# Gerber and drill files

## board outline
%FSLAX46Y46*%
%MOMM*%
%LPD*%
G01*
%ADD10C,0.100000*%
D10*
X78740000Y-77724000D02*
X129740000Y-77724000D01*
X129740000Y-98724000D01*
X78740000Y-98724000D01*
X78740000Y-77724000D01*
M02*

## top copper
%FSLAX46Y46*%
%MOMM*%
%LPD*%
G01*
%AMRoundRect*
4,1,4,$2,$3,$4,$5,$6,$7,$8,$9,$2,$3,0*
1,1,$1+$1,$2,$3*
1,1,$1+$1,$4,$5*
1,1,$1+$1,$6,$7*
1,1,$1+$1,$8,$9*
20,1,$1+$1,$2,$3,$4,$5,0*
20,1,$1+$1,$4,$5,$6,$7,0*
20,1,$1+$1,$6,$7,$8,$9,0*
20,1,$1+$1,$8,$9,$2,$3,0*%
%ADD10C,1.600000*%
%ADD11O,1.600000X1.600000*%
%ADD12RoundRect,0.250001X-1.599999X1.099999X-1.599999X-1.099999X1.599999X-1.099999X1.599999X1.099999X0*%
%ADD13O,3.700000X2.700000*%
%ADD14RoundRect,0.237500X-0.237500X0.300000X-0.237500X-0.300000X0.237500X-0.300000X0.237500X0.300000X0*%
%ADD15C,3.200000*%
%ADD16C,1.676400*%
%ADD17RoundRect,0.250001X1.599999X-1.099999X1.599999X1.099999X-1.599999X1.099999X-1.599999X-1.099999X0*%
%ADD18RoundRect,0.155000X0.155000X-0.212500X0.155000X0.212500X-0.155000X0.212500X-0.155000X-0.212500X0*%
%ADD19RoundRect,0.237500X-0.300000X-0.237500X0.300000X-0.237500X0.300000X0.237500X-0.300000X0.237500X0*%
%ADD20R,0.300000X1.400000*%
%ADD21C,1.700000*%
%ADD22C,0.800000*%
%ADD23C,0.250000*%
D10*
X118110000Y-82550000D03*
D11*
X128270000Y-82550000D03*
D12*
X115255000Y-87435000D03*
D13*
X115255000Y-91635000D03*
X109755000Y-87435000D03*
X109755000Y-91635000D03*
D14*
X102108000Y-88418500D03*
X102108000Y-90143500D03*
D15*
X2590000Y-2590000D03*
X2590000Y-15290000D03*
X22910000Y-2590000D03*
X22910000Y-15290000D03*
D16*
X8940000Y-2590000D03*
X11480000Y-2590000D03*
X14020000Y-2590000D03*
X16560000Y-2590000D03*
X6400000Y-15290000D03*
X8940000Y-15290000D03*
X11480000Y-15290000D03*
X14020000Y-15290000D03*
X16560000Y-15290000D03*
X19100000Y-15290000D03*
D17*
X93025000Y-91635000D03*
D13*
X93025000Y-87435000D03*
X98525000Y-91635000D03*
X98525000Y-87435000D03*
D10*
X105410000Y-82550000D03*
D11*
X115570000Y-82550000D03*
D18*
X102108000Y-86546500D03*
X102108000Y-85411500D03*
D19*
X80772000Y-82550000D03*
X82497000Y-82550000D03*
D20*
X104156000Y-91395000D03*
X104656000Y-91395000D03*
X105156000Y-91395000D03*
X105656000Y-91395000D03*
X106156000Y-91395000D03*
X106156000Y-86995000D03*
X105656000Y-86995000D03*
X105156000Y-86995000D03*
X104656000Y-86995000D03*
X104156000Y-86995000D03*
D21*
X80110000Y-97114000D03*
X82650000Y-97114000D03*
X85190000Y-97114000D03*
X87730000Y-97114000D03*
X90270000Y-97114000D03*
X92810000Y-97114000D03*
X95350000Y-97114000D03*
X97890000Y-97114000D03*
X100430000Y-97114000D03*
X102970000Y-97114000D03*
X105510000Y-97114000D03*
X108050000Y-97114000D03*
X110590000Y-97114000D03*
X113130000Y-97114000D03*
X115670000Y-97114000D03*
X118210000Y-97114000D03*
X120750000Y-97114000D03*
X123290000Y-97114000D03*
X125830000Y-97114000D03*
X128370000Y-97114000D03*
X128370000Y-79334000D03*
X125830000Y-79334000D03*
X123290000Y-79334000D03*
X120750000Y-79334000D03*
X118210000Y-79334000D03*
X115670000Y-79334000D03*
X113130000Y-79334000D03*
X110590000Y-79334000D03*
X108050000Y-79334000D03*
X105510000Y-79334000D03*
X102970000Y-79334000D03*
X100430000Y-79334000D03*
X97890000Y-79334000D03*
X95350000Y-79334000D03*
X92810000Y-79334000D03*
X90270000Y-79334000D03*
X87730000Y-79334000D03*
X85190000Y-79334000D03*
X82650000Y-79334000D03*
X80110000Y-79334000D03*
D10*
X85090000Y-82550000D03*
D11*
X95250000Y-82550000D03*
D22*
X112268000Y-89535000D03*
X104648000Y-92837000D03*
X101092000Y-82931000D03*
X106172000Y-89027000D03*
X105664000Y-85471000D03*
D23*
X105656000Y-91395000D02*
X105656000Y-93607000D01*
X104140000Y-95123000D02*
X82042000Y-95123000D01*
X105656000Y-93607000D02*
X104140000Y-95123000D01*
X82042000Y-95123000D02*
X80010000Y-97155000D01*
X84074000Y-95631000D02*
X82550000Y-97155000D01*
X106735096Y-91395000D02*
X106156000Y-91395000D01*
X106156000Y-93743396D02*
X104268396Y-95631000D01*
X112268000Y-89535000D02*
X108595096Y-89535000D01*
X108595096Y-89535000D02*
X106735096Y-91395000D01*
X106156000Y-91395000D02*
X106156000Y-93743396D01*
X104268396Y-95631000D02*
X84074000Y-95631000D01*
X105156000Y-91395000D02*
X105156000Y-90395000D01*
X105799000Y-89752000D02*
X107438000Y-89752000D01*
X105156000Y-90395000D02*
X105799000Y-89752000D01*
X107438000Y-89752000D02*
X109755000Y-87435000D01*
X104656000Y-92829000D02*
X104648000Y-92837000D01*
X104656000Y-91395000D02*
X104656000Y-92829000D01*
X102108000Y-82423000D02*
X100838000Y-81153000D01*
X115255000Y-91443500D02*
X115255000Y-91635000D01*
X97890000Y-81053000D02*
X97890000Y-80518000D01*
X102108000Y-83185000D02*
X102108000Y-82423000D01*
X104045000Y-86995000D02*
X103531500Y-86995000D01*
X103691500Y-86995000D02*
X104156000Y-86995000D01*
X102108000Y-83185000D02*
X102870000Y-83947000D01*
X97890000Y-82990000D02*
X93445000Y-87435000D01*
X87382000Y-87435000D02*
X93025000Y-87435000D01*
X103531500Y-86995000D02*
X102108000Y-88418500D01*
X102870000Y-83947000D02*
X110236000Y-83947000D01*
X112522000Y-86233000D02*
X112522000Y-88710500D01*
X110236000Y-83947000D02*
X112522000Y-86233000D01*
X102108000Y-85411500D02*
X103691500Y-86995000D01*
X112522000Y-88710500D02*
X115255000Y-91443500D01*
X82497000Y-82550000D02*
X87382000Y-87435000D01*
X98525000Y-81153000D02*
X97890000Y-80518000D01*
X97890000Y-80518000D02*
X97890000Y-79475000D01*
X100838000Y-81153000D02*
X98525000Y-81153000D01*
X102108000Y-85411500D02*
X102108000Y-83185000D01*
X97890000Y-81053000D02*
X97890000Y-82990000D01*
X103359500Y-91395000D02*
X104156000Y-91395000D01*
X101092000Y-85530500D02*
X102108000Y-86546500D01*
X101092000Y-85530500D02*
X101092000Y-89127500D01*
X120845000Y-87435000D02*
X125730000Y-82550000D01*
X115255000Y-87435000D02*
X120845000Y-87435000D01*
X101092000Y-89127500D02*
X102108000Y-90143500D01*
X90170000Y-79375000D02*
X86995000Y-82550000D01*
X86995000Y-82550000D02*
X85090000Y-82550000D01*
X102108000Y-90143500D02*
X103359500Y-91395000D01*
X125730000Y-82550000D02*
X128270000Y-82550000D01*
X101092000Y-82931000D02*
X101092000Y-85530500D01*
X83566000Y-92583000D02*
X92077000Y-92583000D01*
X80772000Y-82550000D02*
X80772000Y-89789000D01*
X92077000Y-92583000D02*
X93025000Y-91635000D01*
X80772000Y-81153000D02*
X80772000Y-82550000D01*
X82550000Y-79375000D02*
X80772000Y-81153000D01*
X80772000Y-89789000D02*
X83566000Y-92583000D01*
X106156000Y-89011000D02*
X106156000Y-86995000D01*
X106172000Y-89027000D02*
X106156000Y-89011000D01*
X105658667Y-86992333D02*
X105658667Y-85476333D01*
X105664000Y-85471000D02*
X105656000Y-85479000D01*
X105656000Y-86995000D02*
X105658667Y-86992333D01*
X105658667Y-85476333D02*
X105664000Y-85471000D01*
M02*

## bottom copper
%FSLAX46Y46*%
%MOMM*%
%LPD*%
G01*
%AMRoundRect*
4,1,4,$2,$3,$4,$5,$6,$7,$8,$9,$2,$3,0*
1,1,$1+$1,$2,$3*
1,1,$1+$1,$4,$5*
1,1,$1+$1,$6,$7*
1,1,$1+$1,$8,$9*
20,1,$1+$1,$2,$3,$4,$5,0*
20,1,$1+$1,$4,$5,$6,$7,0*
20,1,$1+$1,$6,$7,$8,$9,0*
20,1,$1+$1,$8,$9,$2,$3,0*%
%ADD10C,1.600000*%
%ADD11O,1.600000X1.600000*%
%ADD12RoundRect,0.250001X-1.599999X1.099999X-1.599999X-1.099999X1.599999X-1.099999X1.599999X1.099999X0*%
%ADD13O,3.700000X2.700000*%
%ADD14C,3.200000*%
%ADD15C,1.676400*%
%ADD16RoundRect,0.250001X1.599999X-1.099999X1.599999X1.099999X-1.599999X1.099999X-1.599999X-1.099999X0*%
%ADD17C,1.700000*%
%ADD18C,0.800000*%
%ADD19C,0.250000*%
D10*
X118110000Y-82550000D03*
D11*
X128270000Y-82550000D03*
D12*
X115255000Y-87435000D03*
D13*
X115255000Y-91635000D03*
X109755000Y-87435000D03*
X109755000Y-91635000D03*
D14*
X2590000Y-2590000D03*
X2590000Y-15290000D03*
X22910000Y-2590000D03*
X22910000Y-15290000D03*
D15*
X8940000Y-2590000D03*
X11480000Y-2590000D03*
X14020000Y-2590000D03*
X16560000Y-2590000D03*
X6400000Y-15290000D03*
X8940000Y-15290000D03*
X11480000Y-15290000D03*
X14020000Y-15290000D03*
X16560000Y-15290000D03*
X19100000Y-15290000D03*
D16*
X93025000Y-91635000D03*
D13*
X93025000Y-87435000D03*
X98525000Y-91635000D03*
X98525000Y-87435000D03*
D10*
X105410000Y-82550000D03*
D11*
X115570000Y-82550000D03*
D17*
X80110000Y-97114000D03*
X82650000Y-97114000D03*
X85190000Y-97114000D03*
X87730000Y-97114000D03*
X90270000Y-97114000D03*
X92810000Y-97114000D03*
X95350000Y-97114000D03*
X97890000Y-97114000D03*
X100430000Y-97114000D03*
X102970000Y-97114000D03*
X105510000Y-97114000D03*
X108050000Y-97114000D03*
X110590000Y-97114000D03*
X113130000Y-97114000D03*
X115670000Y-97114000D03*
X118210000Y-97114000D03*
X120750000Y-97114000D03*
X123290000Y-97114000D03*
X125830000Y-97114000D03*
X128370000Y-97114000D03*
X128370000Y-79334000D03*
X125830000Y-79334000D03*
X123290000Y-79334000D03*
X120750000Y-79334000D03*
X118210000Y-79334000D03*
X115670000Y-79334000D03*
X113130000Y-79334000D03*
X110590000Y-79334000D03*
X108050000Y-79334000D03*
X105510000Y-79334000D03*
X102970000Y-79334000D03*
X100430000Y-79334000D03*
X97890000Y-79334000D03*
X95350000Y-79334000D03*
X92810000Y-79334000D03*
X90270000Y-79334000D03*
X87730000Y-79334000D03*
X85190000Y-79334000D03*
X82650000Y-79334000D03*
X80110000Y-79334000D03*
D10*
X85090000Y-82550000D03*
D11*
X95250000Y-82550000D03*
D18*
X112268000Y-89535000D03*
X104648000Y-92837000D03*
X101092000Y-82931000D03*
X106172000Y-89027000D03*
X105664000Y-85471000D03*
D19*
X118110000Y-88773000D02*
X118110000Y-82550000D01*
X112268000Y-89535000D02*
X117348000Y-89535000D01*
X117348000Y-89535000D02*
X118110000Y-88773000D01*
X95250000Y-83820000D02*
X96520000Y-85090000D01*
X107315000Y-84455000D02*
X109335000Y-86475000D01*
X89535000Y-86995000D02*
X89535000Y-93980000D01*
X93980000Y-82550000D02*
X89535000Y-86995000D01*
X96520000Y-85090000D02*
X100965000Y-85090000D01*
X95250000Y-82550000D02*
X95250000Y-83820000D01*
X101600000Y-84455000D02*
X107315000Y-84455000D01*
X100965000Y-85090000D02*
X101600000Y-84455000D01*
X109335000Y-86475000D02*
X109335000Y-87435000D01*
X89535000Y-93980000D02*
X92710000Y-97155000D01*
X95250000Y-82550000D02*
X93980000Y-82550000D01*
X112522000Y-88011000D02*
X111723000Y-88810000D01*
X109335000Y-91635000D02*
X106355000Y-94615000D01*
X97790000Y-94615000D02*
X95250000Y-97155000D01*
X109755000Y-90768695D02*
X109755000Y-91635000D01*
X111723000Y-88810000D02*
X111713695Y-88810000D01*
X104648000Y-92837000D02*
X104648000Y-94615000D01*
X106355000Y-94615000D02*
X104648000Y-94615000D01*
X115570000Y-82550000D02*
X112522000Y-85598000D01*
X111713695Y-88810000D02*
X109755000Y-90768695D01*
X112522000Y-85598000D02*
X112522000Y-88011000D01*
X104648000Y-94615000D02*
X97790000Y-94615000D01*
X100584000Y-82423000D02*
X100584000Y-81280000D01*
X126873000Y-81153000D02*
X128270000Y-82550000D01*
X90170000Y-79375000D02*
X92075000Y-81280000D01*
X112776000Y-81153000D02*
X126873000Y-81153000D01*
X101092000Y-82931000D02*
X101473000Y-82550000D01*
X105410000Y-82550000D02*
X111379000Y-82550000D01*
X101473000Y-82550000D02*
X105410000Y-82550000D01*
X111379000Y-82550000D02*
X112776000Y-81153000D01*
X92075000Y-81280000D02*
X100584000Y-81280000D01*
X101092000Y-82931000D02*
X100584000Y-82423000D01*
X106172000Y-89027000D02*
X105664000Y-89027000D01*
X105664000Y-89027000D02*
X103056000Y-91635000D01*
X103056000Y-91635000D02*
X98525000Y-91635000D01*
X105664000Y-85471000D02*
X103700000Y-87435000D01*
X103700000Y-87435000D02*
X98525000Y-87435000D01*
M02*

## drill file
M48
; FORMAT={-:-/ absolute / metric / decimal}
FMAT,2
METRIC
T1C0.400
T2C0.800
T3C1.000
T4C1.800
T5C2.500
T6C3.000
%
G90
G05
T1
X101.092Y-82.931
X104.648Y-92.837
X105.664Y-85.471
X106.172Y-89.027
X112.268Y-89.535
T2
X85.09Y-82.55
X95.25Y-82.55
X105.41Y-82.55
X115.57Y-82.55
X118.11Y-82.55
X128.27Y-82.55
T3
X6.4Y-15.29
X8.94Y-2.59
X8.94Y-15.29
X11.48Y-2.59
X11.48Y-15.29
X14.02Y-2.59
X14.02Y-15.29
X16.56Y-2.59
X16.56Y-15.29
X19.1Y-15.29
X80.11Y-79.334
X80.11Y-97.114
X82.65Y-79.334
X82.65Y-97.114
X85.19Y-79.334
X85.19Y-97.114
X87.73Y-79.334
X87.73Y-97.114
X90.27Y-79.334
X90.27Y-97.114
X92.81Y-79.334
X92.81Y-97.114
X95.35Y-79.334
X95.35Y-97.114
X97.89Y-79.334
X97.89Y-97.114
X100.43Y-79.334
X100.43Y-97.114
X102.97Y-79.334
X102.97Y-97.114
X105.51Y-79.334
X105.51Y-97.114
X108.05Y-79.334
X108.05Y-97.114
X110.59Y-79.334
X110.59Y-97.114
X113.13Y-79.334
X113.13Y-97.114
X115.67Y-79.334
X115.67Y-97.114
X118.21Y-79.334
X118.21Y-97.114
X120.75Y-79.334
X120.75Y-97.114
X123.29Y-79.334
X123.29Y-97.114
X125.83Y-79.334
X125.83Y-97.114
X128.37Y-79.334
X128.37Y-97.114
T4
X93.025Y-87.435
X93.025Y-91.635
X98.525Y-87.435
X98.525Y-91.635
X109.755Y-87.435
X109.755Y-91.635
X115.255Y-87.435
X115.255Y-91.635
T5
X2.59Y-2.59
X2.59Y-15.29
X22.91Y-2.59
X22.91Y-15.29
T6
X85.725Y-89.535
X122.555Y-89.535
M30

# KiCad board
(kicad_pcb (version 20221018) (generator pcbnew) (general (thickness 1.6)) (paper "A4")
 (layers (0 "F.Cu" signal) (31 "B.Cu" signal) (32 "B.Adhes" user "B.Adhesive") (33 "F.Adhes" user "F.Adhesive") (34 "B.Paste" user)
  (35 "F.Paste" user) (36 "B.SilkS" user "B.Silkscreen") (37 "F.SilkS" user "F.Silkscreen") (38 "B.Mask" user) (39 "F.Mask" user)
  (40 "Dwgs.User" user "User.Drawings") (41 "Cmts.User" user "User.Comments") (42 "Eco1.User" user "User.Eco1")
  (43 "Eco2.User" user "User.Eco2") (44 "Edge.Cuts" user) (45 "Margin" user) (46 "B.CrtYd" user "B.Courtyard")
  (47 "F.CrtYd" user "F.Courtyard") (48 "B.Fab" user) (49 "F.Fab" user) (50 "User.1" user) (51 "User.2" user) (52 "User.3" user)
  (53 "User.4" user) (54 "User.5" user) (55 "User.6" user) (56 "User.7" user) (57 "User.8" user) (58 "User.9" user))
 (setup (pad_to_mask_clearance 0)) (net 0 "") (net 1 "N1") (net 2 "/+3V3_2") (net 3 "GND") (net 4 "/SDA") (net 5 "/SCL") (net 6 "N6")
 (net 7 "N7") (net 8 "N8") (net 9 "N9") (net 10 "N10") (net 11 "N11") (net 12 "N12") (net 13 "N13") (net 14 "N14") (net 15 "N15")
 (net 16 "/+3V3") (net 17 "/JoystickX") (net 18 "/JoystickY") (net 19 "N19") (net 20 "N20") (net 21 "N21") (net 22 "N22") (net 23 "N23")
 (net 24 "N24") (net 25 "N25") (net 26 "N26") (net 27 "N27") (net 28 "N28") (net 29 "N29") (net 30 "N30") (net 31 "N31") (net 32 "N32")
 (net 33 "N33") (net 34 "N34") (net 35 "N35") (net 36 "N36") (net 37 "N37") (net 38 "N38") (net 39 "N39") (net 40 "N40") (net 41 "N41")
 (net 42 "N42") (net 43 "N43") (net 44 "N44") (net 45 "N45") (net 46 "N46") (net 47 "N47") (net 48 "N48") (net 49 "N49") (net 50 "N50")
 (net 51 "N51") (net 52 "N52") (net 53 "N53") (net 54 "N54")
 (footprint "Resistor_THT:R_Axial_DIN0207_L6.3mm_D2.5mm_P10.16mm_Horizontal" (layer "F.Cu") (at 118.11 82.55)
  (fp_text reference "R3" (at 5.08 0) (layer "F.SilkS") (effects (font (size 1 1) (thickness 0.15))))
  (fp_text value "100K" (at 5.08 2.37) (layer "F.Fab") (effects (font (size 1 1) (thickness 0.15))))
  (pad "1" thru_hole circle (at 0 0) (size 1.6 1.6) (drill 0.8) (layers "*.Cu" "*.Mask") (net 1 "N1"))
  (pad "2" thru_hole oval (at 10.16 0) (size 1.6 1.6) (drill 0.8) (layers "*.Cu" "*.Mask") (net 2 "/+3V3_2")))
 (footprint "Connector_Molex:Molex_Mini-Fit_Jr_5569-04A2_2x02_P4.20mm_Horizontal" (layer "F.Cu") (at 115.255 87.435 -90)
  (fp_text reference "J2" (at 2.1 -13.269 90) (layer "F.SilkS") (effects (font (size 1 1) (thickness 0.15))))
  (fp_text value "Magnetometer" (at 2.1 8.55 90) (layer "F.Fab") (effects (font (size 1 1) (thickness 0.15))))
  (pad "" np_thru_hole circle (at 2.1 -7.3 270) (size 3 3) (drill 3) (layers "*.Cu" "*.Mask"))
  (pad "1" thru_hole roundrect (at 0 0 270) (size 2.7 3.7) (drill 1.8) (layers "*.Cu" "*.Mask") (roundrect_rratio 0.092593)
   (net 2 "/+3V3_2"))
  (pad "2" thru_hole oval (at 4.2 0 270) (size 2.7 3.7) (drill 1.8) (layers "*.Cu" "*.Mask") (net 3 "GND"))
  (pad "3" thru_hole oval (at 0 5.5 270) (size 2.7 3.7) (drill 1.8) (layers "*.Cu" "*.Mask") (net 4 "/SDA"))
  (pad "4" thru_hole oval (at 4.2 5.5 270) (size 2.7 3.7) (drill 1.8) (layers "*.Cu" "*.Mask") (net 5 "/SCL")))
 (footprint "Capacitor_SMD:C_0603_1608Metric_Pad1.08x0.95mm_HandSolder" (layer "F.Cu") (at 102.108 89.281 -90)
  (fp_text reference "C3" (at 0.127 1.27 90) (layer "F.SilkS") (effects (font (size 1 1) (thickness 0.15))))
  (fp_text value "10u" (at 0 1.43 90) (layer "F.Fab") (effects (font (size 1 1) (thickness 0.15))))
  (pad "1" smd roundrect (at -0.8625 0 270) (size 1.075 0.95) (layers "F.Cu" "F.Paste" "F.Mask") (roundrect_rratio 0.25) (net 3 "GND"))
  (pad "2" smd roundrect (at 0.8625 0 270) (size 1.075 0.95) (layers "F.Cu" "F.Paste" "F.Mask") (roundrect_rratio 0.25) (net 2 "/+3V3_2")))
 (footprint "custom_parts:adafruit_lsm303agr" (layer "F.Cu") (at 12.75 10.21)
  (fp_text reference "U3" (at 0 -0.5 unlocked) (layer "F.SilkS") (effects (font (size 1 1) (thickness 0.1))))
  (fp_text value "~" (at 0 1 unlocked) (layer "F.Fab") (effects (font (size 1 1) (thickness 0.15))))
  (pad "" thru_hole circle (at -10.16 -7.62) (size 3.2 3.2) (drill 2.5) (layers "*.Cu" "*.Mask") (zone_connect 0))
  (pad "" thru_hole circle (at -10.16 5.08) (size 3.2 3.2) (drill 2.5) (layers "*.Cu" "*.Mask") (zone_connect 0))
  (pad "" thru_hole circle (at 10.16 -7.62) (size 3.2 3.2) (drill 2.5) (layers "*.Cu" "*.Mask") (zone_connect 0))
  (pad "" thru_hole circle (at 10.16 5.08) (size 3.2 3.2) (drill 2.5) (layers "*.Cu" "*.Mask") (zone_connect 0))
  (pad "0" thru_hole circle (at -3.81 -7.62 90) (size 1.6764 1.6764) (drill 1) (layers "*.Cu" "*.Mask") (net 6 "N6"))
  (pad "1" thru_hole circle (at -1.27 -7.62 90) (size 1.6764 1.6764) (drill 1) (layers "*.Cu" "*.Mask") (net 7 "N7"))
  (pad "2" thru_hole circle (at 1.27 -7.62 90) (size 1.6764 1.6764) (drill 1) (layers "*.Cu" "*.Mask") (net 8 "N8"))
  (pad "3" thru_hole circle (at 3.81 -7.62 90) (size 1.6764 1.6764) (drill 1) (layers "*.Cu" "*.Mask") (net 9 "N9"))
  (pad "4" thru_hole circle (at -6.35 5.08 90) (size 1.6764 1.6764) (drill 1) (layers "*.Cu" "*.Mask") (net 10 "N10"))
  (pad "5" thru_hole circle (at -3.81 5.08 90) (size 1.6764 1.6764) (drill 1) (layers "*.Cu" "*.Mask") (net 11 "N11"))
  (pad "6" thru_hole circle (at -1.27 5.08 90) (size 1.6764 1.6764) (drill 1) (layers "*.Cu" "*.Mask") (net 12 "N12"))
  (pad "7" thru_hole circle (at 1.27 5.08 90) (size 1.6764 1.6764) (drill 1) (layers "*.Cu" "*.Mask") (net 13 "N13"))
  (pad "8" thru_hole circle (at 3.81 5.08 90) (size 1.6764 1.6764) (drill 1) (layers "*.Cu" "*.Mask") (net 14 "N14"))
  (pad "9" thru_hole circle (at 6.35 5.08 90) (size 1.6764 1.6764) (drill 1) (layers "*.Cu" "*.Mask") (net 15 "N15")))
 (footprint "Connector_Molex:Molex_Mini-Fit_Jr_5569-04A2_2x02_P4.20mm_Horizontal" (layer "F.Cu") (at 93.025 91.635 90)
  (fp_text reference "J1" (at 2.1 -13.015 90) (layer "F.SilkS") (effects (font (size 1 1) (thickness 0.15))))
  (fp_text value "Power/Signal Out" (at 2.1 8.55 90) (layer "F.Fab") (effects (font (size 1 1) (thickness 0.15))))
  (pad "" np_thru_hole circle (at 2.1 -7.3 90) (size 3 3) (drill 3) (layers "*.Cu" "*.Mask"))
  (pad "1" thru_hole roundrect (at 0 0 90) (size 2.7 3.7) (drill 1.8) (layers "*.Cu" "*.Mask") (roundrect_rratio 0.092593) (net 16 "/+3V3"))
  (pad "2" thru_hole oval (at 4.2 0 90) (size 2.7 3.7) (drill 1.8) (layers "*.Cu" "*.Mask") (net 3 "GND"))
  (pad "3" thru_hole oval (at 0 5.5 90) (size 2.7 3.7) (drill 1.8) (layers "*.Cu" "*.Mask") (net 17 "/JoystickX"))
  (pad "4" thru_hole oval (at 4.2 5.5 90) (size 2.7 3.7) (drill 1.8) (layers "*.Cu" "*.Mask") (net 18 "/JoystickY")))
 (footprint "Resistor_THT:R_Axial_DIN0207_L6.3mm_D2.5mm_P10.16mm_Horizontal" (layer "F.Cu") (at 105.41 82.55)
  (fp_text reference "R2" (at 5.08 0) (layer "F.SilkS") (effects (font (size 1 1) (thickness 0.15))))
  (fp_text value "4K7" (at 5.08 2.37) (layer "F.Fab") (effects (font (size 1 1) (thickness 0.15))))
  (pad "1" thru_hole circle (at 0 0) (size 1.6 1.6) (drill 0.8) (layers "*.Cu" "*.Mask") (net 2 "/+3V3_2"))
  (pad "2" thru_hole oval (at 10.16 0) (size 1.6 1.6) (drill 0.8) (layers "*.Cu" "*.Mask") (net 5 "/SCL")))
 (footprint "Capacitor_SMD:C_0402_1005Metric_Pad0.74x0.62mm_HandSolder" (layer "F.Cu") (at 102.108 85.979 90)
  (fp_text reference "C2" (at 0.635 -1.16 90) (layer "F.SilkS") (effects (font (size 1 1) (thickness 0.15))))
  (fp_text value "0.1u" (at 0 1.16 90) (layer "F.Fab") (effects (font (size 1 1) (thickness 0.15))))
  (pad "1" smd roundrect (at -0.5675 0 90) (size 0.735 0.62) (layers "F.Cu" "F.Paste" "F.Mask") (roundrect_rratio 0.25) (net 2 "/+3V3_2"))
  (pad "2" smd roundrect (at 0.5675 0 90) (size 0.735 0.62) (layers "F.Cu" "F.Paste" "F.Mask") (roundrect_rratio 0.25) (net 3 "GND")))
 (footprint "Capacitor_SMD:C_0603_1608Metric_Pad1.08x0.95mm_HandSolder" (layer "F.Cu") (at 81.6345 82.55)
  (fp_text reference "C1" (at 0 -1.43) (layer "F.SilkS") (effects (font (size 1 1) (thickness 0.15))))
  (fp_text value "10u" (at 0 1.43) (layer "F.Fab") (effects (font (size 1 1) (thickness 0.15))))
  (pad "1" smd roundrect (at -0.8625 0) (size 1.075 0.95) (layers "F.Cu" "F.Paste" "F.Mask") (roundrect_rratio 0.25) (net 16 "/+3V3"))
  (pad "2" smd roundrect (at 0.8625 0) (size 1.075 0.95) (layers "F.Cu" "F.Paste" "F.Mask") (roundrect_rratio 0.25) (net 3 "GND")))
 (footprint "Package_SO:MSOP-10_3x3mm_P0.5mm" (layer "F.Cu") (at 105.156 89.195 90)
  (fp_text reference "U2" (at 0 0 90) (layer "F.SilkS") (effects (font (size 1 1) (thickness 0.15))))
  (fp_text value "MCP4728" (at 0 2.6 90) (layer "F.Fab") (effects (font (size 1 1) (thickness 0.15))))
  (pad "1" smd rect (at -2.2 -1 90) (size 1.4 0.3) (layers "F.Cu" "F.Paste" "F.Mask") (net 2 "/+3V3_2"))
  (pad "2" smd rect (at -2.2 -0.5 90) (size 1.4 0.3) (layers "F.Cu" "F.Paste" "F.Mask") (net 5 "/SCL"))
  (pad "3" smd rect (at -2.2 0 90) (size 1.4 0.3) (layers "F.Cu" "F.Paste" "F.Mask") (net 4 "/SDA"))
  (pad "4" smd rect (at -2.2 0.5 90) (size 1.4 0.3) (layers "F.Cu" "F.Paste" "F.Mask") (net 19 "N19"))
  (pad "5" smd rect (at -2.2 1 90) (size 1.4 0.3) (layers "F.Cu" "F.Paste" "F.Mask") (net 1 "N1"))
  (pad "6" smd rect (at 2.2 1 90) (size 1.4 0.3) (layers "F.Cu" "F.Paste" "F.Mask") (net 17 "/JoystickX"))
  (pad "7" smd rect (at 2.2 0.5 90) (size 1.4 0.3) (layers "F.Cu" "F.Paste" "F.Mask") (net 18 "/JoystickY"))
  (pad "8" smd rect (at 2.2 0 90) (size 1.4 0.3) (layers "F.Cu" "F.Paste" "F.Mask") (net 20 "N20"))
  (pad "9" smd rect (at 2.2 -0.5 90) (size 1.4 0.3) (layers "F.Cu" "F.Paste" "F.Mask") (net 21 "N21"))
  (pad "10" smd rect (at 2.2 -1 90) (size 1.4 0.3) (layers "F.Cu" "F.Paste" "F.Mask") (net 3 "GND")))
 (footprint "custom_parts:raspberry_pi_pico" (layer "F.Cu") (at 103.028 88.606)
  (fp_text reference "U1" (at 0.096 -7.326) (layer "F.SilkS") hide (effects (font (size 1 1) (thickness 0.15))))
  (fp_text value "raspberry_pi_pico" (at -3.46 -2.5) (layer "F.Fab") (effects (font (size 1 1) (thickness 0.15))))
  (pad "1" thru_hole circle (at -22.918 8.508 270) (size 1.7 1.7) (drill 1) (layers "*.Cu" "*.Mask") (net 19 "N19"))
  (pad "2" thru_hole circle (at -20.378 8.508 270) (size 1.7 1.7) (drill 1) (layers "*.Cu" "*.Mask") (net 1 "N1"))
  (pad "3" thru_hole circle (at -17.838 8.508 270) (size 1.7 1.7) (drill 1) (layers "*.Cu" "*.Mask") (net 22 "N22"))
  (pad "4" thru_hole circle (at -15.298 8.508 270) (size 1.7 1.7) (drill 1) (layers "*.Cu" "*.Mask") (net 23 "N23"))
  (pad "5" thru_hole circle (at -12.758 8.508 270) (size 1.7 1.7) (drill 1) (layers "*.Cu" "*.Mask") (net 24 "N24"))
  (pad "6" thru_hole circle (at -10.218 8.508 270) (size 1.7 1.7) (drill 1) (layers "*.Cu" "*.Mask") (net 4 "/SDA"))
  (pad "7" thru_hole circle (at -7.678 8.508 270) (size 1.7 1.7) (drill 1) (layers "*.Cu" "*.Mask") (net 5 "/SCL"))
  (pad "8" thru_hole circle (at -5.138 8.508 270) (size 1.7 1.7) (drill 1) (layers "*.Cu" "*.Mask") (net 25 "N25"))
  (pad "9" thru_hole circle (at -2.598 8.508 270) (size 1.7 1.7) (drill 1) (layers "*.Cu" "*.Mask") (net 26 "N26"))
  (pad "10" thru_hole circle (at -0.058 8.508 270) (size 1.7 1.7) (drill 1) (layers "*.Cu" "*.Mask") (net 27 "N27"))
  (pad "11" thru_hole circle (at 2.482 8.508 270) (size 1.7 1.7) (drill 1) (layers "*.Cu" "*.Mask") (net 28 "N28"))
  (pad "12" thru_hole circle (at 5.022 8.508 270) (size 1.7 1.7) (drill 1) (layers "*.Cu" "*.Mask") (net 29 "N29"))
  (pad "13" thru_hole circle (at 7.562 8.508 270) (size 1.7 1.7) (drill 1) (layers "*.Cu" "*.Mask") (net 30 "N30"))
  (pad "14" thru_hole circle (at 10.102 8.508 270) (size 1.7 1.7) (drill 1) (layers "*.Cu" "*.Mask") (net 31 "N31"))
  (pad "15" thru_hole circle (at 12.642 8.508 270) (size 1.7 1.7) (drill 1) (layers "*.Cu" "*.Mask") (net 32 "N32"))
  (pad "16" thru_hole circle (at 15.182 8.508 270) (size 1.7 1.7) (drill 1) (layers "*.Cu" "*.Mask") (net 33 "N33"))
  (pad "17" thru_hole circle (at 17.722 8.508 270) (size 1.7 1.7) (drill 1) (layers "*.Cu" "*.Mask") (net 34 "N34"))
  (pad "18" thru_hole circle (at 20.262 8.508 270) (size 1.7 1.7) (drill 1) (layers "*.Cu" "*.Mask") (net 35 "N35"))
  (pad "19" thru_hole circle (at 22.802 8.508 270) (size 1.7 1.7) (drill 1) (layers "*.Cu" "*.Mask") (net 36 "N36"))
  (pad "20" thru_hole circle (at 25.342 8.508 270) (size 1.7 1.7) (drill 1) (layers "*.Cu" "*.Mask") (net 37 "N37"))
  (pad "21" thru_hole circle (at 25.342 -9.272 270) (size 1.7 1.7) (drill 1) (layers "*.Cu" "*.Mask") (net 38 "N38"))
  (pad "22" thru_hole circle (at 22.802 -9.272 270) (size 1.7 1.7) (drill 1) (layers "*.Cu" "*.Mask") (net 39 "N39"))
  (pad "23" thru_hole circle (at 20.262 -9.272 270) (size 1.7 1.7) (drill 1) (layers "*.Cu" "*.Mask") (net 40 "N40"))
  (pad "24" thru_hole circle (at 17.722 -9.272 270) (size 1.7 1.7) (drill 1) (layers "*.Cu" "*.Mask") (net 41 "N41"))
  (pad "25" thru_hole circle (at 15.182 -9.272 270) (size 1.7 1.7) (drill 1) (layers "*.Cu" "*.Mask") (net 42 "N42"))
  (pad "26" thru_hole circle (at 12.642 -9.272 270) (size 1.7 1.7) (drill 1) (layers "*.Cu" "*.Mask") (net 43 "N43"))
  (pad "27" thru_hole circle (at 10.102 -9.272 270) (size 1.7 1.7) (drill 1) (layers "*.Cu" "*.Mask") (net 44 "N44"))
  (pad "28" thru_hole circle (at 7.562 -9.272 270) (size 1.7 1.7) (drill 1) (layers "*.Cu" "*.Mask") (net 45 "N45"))
  (pad "29" thru_hole circle (at 5.022 -9.272 270) (size 1.7 1.7) (drill 1) (layers "*.Cu" "*.Mask") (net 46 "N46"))
  (pad "30" thru_hole circle (at 2.482 -9.272 270) (size 1.7 1.7) (drill 1) (layers "*.Cu" "*.Mask") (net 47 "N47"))
  (pad "31" thru_hole circle (at -0.058 -9.272 270) (size 1.7 1.7) (drill 1) (layers "*.Cu" "*.Mask") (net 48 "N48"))
  (pad "32" thru_hole circle (at -2.598 -9.272 270) (size 1.7 1.7) (drill 1) (layers "*.Cu" "*.Mask") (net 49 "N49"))
  (pad "33" thru_hole circle (at -5.138 -9.272 270) (size 1.7 1.7) (drill 1) (layers "*.Cu" "*.Mask") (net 3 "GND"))
  (pad "34" thru_hole circle (at -7.678 -9.272 270) (size 1.7 1.7) (drill 1) (layers "*.Cu" "*.Mask") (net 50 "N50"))
  (pad "35" thru_hole circle (at -10.218 -9.272 270) (size 1.7 1.7) (drill 1) (layers "*.Cu" "*.Mask") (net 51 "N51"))
  (pad "36" thru_hole circle (at -12.758 -9.272 270) (size 1.7 1.7) (drill 1) (layers "*.Cu" "*.Mask") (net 2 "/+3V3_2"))
  (pad "37" thru_hole circle (at -15.298 -9.272 270) (size 1.7 1.7) (drill 1) (layers "*.Cu" "*.Mask") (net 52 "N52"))
  (pad "38" thru_hole circle (at -17.838 -9.272 270) (size 1.7 1.7) (drill 1) (layers "*.Cu" "*.Mask") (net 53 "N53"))
  (pad "39" thru_hole circle (at -20.378 -9.272 270) (size 1.7 1.7) (drill 1) (layers "*.Cu" "*.Mask") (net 16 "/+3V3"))
  (pad "40" thru_hole circle (at -22.918 -9.272 270) (size 1.7 1.7) (drill 1) (layers "*.Cu" "*.Mask") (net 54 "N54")))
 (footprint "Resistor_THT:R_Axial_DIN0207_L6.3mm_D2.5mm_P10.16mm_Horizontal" (layer "F.Cu") (at 85.09 82.55)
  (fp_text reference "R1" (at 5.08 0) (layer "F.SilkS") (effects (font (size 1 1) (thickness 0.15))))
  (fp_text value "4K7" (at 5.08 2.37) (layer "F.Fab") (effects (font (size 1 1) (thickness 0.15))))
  (pad "1" thru_hole circle (at 0 0) (size 1.6 1.6) (drill 0.8) (layers "*.Cu" "*.Mask") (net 2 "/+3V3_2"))
  (pad "2" thru_hole oval (at 10.16 0) (size 1.6 1.6) (drill 0.8) (layers "*.Cu" "*.Mask") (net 4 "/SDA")))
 (gr_rect (start 78.74 77.724) (end 129.74 98.724) (stroke (width 0.1) (type solid)) (fill none) (layer "Edge.Cuts"))
 (segment (start 105.656 91.395) (end 105.656 93.607) (width 0.25) (layer "F.Cu") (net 19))
 (segment (start 104.14 95.123) (end 82.042 95.123) (width 0.25) (layer "F.Cu") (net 19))
 (segment (start 105.656 93.607) (end 104.14 95.123) (width 0.25) (layer "F.Cu") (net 19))
 (segment (start 82.042 95.123) (end 80.01 97.155) (width 0.25) (layer "F.Cu") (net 19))
 (segment (start 84.074 95.631) (end 82.55 97.155) (width 0.25) (layer "F.Cu") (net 1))
 (segment (start 106.735096 91.395) (end 106.156 91.395) (width 0.25) (layer "F.Cu") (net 1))
 (segment (start 106.156 93.743396) (end 104.268396 95.631) (width 0.25) (layer "F.Cu") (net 1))
 (segment (start 112.268 89.535) (end 108.595096 89.535) (width 0.25) (layer "F.Cu") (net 1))
 (segment (start 108.595096 89.535) (end 106.735096 91.395) (width 0.25) (layer "F.Cu") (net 1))
 (segment (start 106.156 91.395) (end 106.156 93.743396) (width 0.25) (layer "F.Cu") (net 1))
 (segment (start 104.268396 95.631) (end 84.074 95.631) (width 0.25) (layer "F.Cu") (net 1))
 (via (at 112.268 89.535) (size 0.8) (drill 0.4) (layers "F.Cu" "B.Cu") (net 1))
 (segment (start 118.11 88.773) (end 118.11 82.55) (width 0.25) (layer "B.Cu") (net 1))
 (segment (start 112.268 89.535) (end 117.348 89.535) (width 0.25) (layer "B.Cu") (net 1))
 (segment (start 117.348 89.535) (end 118.11 88.773) (width 0.25) (layer "B.Cu") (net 1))
 (segment (start 105.156 91.395) (end 105.156 90.395) (width 0.25) (layer "F.Cu") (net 4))
 (segment (start 105.799 89.752) (end 107.438 89.752) (width 0.25) (layer "F.Cu") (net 4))
 (segment (start 105.156 90.395) (end 105.799 89.752) (width 0.25) (layer "F.Cu") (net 4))
 (segment (start 107.438 89.752) (end 109.755 87.435) (width 0.25) (layer "F.Cu") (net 4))
 (segment (start 95.25 83.82) (end 96.52 85.09) (width 0.25) (layer "B.Cu") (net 4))
 (segment (start 107.315 84.455) (end 109.335 86.475) (width 0.25) (layer "B.Cu") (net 4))
 (segment (start 89.535 86.995) (end 89.535 93.98) (width 0.25) (layer "B.Cu") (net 4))
 (segment (start 93.98 82.55) (end 89.535 86.995) (width 0.25) (layer "B.Cu") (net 4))
 (segment (start 96.52 85.09) (end 100.965 85.09) (width 0.25) (layer "B.Cu") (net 4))
 (segment (start 95.25 82.55) (end 95.25 83.82) (width 0.25) (layer "B.Cu") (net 4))
 (segment (start 101.6 84.455) (end 107.315 84.455) (width 0.25) (layer "B.Cu") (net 4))
 (segment (start 100.965 85.09) (end 101.6 84.455) (width 0.25) (layer "B.Cu") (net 4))
 (segment (start 109.335 86.475) (end 109.335 87.435) (width 0.25) (layer "B.Cu") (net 4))
 (segment (start 89.535 93.98) (end 92.71 97.155) (width 0.25) (layer "B.Cu") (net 4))
 (segment (start 95.25 82.55) (end 93.98 82.55) (width 0.25) (layer "B.Cu") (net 4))
 (segment (start 104.656 92.829) (end 104.648 92.837) (width 0.25) (layer "F.Cu") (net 5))
 (segment (start 104.656 91.395) (end 104.656 92.829) (width 0.25) (layer "F.Cu") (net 5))
 (via (at 104.648 92.837) (size 0.8) (drill 0.4) (layers "F.Cu" "B.Cu") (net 5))
 (segment (start 112.522 88.011) (end 111.723 88.81) (width 0.25) (layer "B.Cu") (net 5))
 (segment (start 109.335 91.635) (end 106.355 94.615) (width 0.25) (layer "B.Cu") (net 5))
 (segment (start 97.79 94.615) (end 95.25 97.155) (width 0.25) (layer "B.Cu") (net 5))
 (segment (start 109.755 90.768695) (end 109.755 91.635) (width 0.25) (layer "B.Cu") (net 5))
 (segment (start 111.723 88.81) (end 111.713695 88.81) (width 0.25) (layer "B.Cu") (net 5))
 (segment (start 104.648 92.837) (end 104.648 94.615) (width 0.25) (layer "B.Cu") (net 5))
 (segment (start 106.355 94.615) (end 104.648 94.615) (width 0.25) (layer "B.Cu") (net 5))
 (segment (start 115.57 82.55) (end 112.522 85.598) (width 0.25) (layer "B.Cu") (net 5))
 (segment (start 111.713695 88.81) (end 109.755 90.768695) (width 0.25) (layer "B.Cu") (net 5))
 (segment (start 112.522 85.598) (end 112.522 88.011) (width 0.25) (layer "B.Cu") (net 5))
 (segment (start 104.648 94.615) (end 97.79 94.615) (width 0.25) (layer "B.Cu") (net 5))
 (segment (start 102.108 82.423) (end 100.838 81.153) (width 0.25) (layer "F.Cu") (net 3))
 (segment (start 115.255 91.4435) (end 115.255 91.635) (width 0.25) (layer "F.Cu") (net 3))
 (segment (start 97.89 81.053) (end 97.89 80.518) (width 0.25) (layer "F.Cu") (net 3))
 (segment (start 102.108 83.185) (end 102.108 82.423) (width 0.25) (layer "F.Cu") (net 3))
 (segment (start 104.045 86.995) (end 103.5315 86.995) (width 0.25) (layer "F.Cu") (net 3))
 (segment (start 103.6915 86.995) (end 104.156 86.995) (width 0.25) (layer "F.Cu") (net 3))
 (segment (start 102.108 83.185) (end 102.87 83.947) (width 0.25) (layer "F.Cu") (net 3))
 (segment (start 97.89 82.99) (end 93.445 87.435) (width 0.25) (layer "F.Cu") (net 3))
 (segment (start 87.382 87.435) (end 93.025 87.435) (width 0.25) (layer "F.Cu") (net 3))
 (segment (start 103.5315 86.995) (end 102.108 88.4185) (width 0.25) (layer "F.Cu") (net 3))
 (segment (start 102.87 83.947) (end 110.236 83.947) (width 0.25) (layer "F.Cu") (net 3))
 (segment (start 112.522 86.233) (end 112.522 88.7105) (width 0.25) (layer "F.Cu") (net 3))
 (segment (start 110.236 83.947) (end 112.522 86.233) (width 0.25) (layer "F.Cu") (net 3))
 (segment (start 102.108 85.4115) (end 103.6915 86.995) (width 0.25) (layer "F.Cu") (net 3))
 (segment (start 112.522 88.7105) (end 115.255 91.4435) (width 0.25) (layer "F.Cu") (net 3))
 (segment (start 82.497 82.55) (end 87.382 87.435) (width 0.25) (layer "F.Cu") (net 3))
 (segment (start 98.525 81.153) (end 97.89 80.518) (width 0.25) (layer "F.Cu") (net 3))
 (segment (start 97.89 80.518) (end 97.89 79.475) (width 0.25) (layer "F.Cu") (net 3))
 (segment (start 100.838 81.153) (end 98.525 81.153) (width 0.25) (layer "F.Cu") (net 3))
 (segment (start 102.108 85.4115) (end 102.108 83.185) (width 0.25) (layer "F.Cu") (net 3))
 (segment (start 97.89 81.053) (end 97.89 82.99) (width 0.25) (layer "F.Cu") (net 3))
 (segment (start 103.3595 91.395) (end 104.156 91.395) (width 0.25) (layer "F.Cu") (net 2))
 (segment (start 101.092 85.5305) (end 102.108 86.5465) (width 0.25) (layer "F.Cu") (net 2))
 (segment (start 101.092 85.5305) (end 101.092 89.1275) (width 0.25) (layer "F.Cu") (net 2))
 (segment (start 120.845 87.435) (end 125.73 82.55) (width 0.25) (layer "F.Cu") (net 2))
 (segment (start 115.255 87.435) (end 120.845 87.435) (width 0.25) (layer "F.Cu") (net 2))
 (segment (start 101.092 89.1275) (end 102.108 90.1435) (width 0.25) (layer "F.Cu") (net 2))
 (segment (start 90.17 79.375) (end 86.995 82.55) (width 0.25) (layer "F.Cu") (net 2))
 (segment (start 86.995 82.55) (end 85.09 82.55) (width 0.25) (layer "F.Cu") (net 2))
 (segment (start 102.108 90.1435) (end 103.3595 91.395) (width 0.25) (layer "F.Cu") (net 2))
 (segment (start 125.73 82.55) (end 128.27 82.55) (width 0.25) (layer "F.Cu") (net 2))
 (segment (start 101.092 82.931) (end 101.092 85.5305) (width 0.25) (layer "F.Cu") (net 2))
 (via (at 101.092 82.931) (size 0.8) (drill 0.4) (layers "F.Cu" "B.Cu") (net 2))
 (segment (start 100.584 82.423) (end 100.584 81.28) (width 0.25) (layer "B.Cu") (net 2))
 (segment (start 126.873 81.153) (end 128.27 82.55) (width 0.25) (layer "B.Cu") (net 2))
 (segment (start 90.17 79.375) (end 92.075 81.28) (width 0.25) (layer "B.Cu") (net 2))
 (segment (start 112.776 81.153) (end 126.873 81.153) (width 0.25) (layer "B.Cu") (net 2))
 (segment (start 101.092 82.931) (end 101.473 82.55) (width 0.25) (layer "B.Cu") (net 2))
 (segment (start 105.41 82.55) (end 111.379 82.55) (width 0.25) (layer "B.Cu") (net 2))
 (segment (start 101.473 82.55) (end 105.41 82.55) (width 0.25) (layer "B.Cu") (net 2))
 (segment (start 111.379 82.55) (end 112.776 81.153) (width 0.25) (layer "B.Cu") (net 2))
 (segment (start 92.075 81.28) (end 100.584 81.28) (width 0.25) (layer "B.Cu") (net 2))
 (segment (start 101.092 82.931) (end 100.584 82.423) (width 0.25) (layer "B.Cu") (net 2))
 (segment (start 83.566 92.583) (end 92.077 92.583) (width 0.25) (layer "F.Cu") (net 16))
 (segment (start 80.772 82.55) (end 80.772 89.789) (width 0.25) (layer "F.Cu") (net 16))
 (segment (start 92.077 92.583) (end 93.025 91.635) (width 0.25) (layer "F.Cu") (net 16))
 (segment (start 80.772 81.153) (end 80.772 82.55) (width 0.25) (layer "F.Cu") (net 16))
 (segment (start 82.55 79.375) (end 80.772 81.153) (width 0.25) (layer "F.Cu") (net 16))
 (segment (start 80.772 89.789) (end 83.566 92.583) (width 0.25) (layer "F.Cu") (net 16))
 (segment (start 106.156 89.011) (end 106.156 86.995) (width 0.25) (layer "F.Cu") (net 17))
 (segment (start 106.172 89.027) (end 106.156 89.011) (width 0.25) (layer "F.Cu") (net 17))
 (via (at 106.172 89.027) (size 0.8) (drill 0.4) (layers "F.Cu" "B.Cu") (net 17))
 (segment (start 106.172 89.027) (end 105.664 89.027) (width 0.25) (layer "B.Cu") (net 17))
 (segment (start 105.664 89.027) (end 103.056 91.635) (width 0.25) (layer "B.Cu") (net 17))
 (segment (start 103.056 91.635) (end 98.525 91.635) (width 0.25) (layer "B.Cu") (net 17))
 (segment (start 105.658667 86.992333) (end 105.658667 85.476333) (width 0.25) (layer "F.Cu") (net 18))
 (segment (start 105.664 85.471) (end 105.656 85.479) (width 0.25) (layer "F.Cu") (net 18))
 (segment (start 105.656 86.995) (end 105.658667 86.992333) (width 0.25) (layer "F.Cu") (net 18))
 (segment (start 105.658667 85.476333) (end 105.664 85.471) (width 0.25) (layer "F.Cu") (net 18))
 (via (at 105.664 85.471) (size 0.8) (drill 0.4) (layers "F.Cu" "B.Cu") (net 18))
 (segment (start 105.664 85.471) (end 103.7 87.435) (width 0.25) (layer "B.Cu") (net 18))
 (segment (start 103.7 87.435) (end 98.525 87.435) (width 0.25) (layer "B.Cu") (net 18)))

